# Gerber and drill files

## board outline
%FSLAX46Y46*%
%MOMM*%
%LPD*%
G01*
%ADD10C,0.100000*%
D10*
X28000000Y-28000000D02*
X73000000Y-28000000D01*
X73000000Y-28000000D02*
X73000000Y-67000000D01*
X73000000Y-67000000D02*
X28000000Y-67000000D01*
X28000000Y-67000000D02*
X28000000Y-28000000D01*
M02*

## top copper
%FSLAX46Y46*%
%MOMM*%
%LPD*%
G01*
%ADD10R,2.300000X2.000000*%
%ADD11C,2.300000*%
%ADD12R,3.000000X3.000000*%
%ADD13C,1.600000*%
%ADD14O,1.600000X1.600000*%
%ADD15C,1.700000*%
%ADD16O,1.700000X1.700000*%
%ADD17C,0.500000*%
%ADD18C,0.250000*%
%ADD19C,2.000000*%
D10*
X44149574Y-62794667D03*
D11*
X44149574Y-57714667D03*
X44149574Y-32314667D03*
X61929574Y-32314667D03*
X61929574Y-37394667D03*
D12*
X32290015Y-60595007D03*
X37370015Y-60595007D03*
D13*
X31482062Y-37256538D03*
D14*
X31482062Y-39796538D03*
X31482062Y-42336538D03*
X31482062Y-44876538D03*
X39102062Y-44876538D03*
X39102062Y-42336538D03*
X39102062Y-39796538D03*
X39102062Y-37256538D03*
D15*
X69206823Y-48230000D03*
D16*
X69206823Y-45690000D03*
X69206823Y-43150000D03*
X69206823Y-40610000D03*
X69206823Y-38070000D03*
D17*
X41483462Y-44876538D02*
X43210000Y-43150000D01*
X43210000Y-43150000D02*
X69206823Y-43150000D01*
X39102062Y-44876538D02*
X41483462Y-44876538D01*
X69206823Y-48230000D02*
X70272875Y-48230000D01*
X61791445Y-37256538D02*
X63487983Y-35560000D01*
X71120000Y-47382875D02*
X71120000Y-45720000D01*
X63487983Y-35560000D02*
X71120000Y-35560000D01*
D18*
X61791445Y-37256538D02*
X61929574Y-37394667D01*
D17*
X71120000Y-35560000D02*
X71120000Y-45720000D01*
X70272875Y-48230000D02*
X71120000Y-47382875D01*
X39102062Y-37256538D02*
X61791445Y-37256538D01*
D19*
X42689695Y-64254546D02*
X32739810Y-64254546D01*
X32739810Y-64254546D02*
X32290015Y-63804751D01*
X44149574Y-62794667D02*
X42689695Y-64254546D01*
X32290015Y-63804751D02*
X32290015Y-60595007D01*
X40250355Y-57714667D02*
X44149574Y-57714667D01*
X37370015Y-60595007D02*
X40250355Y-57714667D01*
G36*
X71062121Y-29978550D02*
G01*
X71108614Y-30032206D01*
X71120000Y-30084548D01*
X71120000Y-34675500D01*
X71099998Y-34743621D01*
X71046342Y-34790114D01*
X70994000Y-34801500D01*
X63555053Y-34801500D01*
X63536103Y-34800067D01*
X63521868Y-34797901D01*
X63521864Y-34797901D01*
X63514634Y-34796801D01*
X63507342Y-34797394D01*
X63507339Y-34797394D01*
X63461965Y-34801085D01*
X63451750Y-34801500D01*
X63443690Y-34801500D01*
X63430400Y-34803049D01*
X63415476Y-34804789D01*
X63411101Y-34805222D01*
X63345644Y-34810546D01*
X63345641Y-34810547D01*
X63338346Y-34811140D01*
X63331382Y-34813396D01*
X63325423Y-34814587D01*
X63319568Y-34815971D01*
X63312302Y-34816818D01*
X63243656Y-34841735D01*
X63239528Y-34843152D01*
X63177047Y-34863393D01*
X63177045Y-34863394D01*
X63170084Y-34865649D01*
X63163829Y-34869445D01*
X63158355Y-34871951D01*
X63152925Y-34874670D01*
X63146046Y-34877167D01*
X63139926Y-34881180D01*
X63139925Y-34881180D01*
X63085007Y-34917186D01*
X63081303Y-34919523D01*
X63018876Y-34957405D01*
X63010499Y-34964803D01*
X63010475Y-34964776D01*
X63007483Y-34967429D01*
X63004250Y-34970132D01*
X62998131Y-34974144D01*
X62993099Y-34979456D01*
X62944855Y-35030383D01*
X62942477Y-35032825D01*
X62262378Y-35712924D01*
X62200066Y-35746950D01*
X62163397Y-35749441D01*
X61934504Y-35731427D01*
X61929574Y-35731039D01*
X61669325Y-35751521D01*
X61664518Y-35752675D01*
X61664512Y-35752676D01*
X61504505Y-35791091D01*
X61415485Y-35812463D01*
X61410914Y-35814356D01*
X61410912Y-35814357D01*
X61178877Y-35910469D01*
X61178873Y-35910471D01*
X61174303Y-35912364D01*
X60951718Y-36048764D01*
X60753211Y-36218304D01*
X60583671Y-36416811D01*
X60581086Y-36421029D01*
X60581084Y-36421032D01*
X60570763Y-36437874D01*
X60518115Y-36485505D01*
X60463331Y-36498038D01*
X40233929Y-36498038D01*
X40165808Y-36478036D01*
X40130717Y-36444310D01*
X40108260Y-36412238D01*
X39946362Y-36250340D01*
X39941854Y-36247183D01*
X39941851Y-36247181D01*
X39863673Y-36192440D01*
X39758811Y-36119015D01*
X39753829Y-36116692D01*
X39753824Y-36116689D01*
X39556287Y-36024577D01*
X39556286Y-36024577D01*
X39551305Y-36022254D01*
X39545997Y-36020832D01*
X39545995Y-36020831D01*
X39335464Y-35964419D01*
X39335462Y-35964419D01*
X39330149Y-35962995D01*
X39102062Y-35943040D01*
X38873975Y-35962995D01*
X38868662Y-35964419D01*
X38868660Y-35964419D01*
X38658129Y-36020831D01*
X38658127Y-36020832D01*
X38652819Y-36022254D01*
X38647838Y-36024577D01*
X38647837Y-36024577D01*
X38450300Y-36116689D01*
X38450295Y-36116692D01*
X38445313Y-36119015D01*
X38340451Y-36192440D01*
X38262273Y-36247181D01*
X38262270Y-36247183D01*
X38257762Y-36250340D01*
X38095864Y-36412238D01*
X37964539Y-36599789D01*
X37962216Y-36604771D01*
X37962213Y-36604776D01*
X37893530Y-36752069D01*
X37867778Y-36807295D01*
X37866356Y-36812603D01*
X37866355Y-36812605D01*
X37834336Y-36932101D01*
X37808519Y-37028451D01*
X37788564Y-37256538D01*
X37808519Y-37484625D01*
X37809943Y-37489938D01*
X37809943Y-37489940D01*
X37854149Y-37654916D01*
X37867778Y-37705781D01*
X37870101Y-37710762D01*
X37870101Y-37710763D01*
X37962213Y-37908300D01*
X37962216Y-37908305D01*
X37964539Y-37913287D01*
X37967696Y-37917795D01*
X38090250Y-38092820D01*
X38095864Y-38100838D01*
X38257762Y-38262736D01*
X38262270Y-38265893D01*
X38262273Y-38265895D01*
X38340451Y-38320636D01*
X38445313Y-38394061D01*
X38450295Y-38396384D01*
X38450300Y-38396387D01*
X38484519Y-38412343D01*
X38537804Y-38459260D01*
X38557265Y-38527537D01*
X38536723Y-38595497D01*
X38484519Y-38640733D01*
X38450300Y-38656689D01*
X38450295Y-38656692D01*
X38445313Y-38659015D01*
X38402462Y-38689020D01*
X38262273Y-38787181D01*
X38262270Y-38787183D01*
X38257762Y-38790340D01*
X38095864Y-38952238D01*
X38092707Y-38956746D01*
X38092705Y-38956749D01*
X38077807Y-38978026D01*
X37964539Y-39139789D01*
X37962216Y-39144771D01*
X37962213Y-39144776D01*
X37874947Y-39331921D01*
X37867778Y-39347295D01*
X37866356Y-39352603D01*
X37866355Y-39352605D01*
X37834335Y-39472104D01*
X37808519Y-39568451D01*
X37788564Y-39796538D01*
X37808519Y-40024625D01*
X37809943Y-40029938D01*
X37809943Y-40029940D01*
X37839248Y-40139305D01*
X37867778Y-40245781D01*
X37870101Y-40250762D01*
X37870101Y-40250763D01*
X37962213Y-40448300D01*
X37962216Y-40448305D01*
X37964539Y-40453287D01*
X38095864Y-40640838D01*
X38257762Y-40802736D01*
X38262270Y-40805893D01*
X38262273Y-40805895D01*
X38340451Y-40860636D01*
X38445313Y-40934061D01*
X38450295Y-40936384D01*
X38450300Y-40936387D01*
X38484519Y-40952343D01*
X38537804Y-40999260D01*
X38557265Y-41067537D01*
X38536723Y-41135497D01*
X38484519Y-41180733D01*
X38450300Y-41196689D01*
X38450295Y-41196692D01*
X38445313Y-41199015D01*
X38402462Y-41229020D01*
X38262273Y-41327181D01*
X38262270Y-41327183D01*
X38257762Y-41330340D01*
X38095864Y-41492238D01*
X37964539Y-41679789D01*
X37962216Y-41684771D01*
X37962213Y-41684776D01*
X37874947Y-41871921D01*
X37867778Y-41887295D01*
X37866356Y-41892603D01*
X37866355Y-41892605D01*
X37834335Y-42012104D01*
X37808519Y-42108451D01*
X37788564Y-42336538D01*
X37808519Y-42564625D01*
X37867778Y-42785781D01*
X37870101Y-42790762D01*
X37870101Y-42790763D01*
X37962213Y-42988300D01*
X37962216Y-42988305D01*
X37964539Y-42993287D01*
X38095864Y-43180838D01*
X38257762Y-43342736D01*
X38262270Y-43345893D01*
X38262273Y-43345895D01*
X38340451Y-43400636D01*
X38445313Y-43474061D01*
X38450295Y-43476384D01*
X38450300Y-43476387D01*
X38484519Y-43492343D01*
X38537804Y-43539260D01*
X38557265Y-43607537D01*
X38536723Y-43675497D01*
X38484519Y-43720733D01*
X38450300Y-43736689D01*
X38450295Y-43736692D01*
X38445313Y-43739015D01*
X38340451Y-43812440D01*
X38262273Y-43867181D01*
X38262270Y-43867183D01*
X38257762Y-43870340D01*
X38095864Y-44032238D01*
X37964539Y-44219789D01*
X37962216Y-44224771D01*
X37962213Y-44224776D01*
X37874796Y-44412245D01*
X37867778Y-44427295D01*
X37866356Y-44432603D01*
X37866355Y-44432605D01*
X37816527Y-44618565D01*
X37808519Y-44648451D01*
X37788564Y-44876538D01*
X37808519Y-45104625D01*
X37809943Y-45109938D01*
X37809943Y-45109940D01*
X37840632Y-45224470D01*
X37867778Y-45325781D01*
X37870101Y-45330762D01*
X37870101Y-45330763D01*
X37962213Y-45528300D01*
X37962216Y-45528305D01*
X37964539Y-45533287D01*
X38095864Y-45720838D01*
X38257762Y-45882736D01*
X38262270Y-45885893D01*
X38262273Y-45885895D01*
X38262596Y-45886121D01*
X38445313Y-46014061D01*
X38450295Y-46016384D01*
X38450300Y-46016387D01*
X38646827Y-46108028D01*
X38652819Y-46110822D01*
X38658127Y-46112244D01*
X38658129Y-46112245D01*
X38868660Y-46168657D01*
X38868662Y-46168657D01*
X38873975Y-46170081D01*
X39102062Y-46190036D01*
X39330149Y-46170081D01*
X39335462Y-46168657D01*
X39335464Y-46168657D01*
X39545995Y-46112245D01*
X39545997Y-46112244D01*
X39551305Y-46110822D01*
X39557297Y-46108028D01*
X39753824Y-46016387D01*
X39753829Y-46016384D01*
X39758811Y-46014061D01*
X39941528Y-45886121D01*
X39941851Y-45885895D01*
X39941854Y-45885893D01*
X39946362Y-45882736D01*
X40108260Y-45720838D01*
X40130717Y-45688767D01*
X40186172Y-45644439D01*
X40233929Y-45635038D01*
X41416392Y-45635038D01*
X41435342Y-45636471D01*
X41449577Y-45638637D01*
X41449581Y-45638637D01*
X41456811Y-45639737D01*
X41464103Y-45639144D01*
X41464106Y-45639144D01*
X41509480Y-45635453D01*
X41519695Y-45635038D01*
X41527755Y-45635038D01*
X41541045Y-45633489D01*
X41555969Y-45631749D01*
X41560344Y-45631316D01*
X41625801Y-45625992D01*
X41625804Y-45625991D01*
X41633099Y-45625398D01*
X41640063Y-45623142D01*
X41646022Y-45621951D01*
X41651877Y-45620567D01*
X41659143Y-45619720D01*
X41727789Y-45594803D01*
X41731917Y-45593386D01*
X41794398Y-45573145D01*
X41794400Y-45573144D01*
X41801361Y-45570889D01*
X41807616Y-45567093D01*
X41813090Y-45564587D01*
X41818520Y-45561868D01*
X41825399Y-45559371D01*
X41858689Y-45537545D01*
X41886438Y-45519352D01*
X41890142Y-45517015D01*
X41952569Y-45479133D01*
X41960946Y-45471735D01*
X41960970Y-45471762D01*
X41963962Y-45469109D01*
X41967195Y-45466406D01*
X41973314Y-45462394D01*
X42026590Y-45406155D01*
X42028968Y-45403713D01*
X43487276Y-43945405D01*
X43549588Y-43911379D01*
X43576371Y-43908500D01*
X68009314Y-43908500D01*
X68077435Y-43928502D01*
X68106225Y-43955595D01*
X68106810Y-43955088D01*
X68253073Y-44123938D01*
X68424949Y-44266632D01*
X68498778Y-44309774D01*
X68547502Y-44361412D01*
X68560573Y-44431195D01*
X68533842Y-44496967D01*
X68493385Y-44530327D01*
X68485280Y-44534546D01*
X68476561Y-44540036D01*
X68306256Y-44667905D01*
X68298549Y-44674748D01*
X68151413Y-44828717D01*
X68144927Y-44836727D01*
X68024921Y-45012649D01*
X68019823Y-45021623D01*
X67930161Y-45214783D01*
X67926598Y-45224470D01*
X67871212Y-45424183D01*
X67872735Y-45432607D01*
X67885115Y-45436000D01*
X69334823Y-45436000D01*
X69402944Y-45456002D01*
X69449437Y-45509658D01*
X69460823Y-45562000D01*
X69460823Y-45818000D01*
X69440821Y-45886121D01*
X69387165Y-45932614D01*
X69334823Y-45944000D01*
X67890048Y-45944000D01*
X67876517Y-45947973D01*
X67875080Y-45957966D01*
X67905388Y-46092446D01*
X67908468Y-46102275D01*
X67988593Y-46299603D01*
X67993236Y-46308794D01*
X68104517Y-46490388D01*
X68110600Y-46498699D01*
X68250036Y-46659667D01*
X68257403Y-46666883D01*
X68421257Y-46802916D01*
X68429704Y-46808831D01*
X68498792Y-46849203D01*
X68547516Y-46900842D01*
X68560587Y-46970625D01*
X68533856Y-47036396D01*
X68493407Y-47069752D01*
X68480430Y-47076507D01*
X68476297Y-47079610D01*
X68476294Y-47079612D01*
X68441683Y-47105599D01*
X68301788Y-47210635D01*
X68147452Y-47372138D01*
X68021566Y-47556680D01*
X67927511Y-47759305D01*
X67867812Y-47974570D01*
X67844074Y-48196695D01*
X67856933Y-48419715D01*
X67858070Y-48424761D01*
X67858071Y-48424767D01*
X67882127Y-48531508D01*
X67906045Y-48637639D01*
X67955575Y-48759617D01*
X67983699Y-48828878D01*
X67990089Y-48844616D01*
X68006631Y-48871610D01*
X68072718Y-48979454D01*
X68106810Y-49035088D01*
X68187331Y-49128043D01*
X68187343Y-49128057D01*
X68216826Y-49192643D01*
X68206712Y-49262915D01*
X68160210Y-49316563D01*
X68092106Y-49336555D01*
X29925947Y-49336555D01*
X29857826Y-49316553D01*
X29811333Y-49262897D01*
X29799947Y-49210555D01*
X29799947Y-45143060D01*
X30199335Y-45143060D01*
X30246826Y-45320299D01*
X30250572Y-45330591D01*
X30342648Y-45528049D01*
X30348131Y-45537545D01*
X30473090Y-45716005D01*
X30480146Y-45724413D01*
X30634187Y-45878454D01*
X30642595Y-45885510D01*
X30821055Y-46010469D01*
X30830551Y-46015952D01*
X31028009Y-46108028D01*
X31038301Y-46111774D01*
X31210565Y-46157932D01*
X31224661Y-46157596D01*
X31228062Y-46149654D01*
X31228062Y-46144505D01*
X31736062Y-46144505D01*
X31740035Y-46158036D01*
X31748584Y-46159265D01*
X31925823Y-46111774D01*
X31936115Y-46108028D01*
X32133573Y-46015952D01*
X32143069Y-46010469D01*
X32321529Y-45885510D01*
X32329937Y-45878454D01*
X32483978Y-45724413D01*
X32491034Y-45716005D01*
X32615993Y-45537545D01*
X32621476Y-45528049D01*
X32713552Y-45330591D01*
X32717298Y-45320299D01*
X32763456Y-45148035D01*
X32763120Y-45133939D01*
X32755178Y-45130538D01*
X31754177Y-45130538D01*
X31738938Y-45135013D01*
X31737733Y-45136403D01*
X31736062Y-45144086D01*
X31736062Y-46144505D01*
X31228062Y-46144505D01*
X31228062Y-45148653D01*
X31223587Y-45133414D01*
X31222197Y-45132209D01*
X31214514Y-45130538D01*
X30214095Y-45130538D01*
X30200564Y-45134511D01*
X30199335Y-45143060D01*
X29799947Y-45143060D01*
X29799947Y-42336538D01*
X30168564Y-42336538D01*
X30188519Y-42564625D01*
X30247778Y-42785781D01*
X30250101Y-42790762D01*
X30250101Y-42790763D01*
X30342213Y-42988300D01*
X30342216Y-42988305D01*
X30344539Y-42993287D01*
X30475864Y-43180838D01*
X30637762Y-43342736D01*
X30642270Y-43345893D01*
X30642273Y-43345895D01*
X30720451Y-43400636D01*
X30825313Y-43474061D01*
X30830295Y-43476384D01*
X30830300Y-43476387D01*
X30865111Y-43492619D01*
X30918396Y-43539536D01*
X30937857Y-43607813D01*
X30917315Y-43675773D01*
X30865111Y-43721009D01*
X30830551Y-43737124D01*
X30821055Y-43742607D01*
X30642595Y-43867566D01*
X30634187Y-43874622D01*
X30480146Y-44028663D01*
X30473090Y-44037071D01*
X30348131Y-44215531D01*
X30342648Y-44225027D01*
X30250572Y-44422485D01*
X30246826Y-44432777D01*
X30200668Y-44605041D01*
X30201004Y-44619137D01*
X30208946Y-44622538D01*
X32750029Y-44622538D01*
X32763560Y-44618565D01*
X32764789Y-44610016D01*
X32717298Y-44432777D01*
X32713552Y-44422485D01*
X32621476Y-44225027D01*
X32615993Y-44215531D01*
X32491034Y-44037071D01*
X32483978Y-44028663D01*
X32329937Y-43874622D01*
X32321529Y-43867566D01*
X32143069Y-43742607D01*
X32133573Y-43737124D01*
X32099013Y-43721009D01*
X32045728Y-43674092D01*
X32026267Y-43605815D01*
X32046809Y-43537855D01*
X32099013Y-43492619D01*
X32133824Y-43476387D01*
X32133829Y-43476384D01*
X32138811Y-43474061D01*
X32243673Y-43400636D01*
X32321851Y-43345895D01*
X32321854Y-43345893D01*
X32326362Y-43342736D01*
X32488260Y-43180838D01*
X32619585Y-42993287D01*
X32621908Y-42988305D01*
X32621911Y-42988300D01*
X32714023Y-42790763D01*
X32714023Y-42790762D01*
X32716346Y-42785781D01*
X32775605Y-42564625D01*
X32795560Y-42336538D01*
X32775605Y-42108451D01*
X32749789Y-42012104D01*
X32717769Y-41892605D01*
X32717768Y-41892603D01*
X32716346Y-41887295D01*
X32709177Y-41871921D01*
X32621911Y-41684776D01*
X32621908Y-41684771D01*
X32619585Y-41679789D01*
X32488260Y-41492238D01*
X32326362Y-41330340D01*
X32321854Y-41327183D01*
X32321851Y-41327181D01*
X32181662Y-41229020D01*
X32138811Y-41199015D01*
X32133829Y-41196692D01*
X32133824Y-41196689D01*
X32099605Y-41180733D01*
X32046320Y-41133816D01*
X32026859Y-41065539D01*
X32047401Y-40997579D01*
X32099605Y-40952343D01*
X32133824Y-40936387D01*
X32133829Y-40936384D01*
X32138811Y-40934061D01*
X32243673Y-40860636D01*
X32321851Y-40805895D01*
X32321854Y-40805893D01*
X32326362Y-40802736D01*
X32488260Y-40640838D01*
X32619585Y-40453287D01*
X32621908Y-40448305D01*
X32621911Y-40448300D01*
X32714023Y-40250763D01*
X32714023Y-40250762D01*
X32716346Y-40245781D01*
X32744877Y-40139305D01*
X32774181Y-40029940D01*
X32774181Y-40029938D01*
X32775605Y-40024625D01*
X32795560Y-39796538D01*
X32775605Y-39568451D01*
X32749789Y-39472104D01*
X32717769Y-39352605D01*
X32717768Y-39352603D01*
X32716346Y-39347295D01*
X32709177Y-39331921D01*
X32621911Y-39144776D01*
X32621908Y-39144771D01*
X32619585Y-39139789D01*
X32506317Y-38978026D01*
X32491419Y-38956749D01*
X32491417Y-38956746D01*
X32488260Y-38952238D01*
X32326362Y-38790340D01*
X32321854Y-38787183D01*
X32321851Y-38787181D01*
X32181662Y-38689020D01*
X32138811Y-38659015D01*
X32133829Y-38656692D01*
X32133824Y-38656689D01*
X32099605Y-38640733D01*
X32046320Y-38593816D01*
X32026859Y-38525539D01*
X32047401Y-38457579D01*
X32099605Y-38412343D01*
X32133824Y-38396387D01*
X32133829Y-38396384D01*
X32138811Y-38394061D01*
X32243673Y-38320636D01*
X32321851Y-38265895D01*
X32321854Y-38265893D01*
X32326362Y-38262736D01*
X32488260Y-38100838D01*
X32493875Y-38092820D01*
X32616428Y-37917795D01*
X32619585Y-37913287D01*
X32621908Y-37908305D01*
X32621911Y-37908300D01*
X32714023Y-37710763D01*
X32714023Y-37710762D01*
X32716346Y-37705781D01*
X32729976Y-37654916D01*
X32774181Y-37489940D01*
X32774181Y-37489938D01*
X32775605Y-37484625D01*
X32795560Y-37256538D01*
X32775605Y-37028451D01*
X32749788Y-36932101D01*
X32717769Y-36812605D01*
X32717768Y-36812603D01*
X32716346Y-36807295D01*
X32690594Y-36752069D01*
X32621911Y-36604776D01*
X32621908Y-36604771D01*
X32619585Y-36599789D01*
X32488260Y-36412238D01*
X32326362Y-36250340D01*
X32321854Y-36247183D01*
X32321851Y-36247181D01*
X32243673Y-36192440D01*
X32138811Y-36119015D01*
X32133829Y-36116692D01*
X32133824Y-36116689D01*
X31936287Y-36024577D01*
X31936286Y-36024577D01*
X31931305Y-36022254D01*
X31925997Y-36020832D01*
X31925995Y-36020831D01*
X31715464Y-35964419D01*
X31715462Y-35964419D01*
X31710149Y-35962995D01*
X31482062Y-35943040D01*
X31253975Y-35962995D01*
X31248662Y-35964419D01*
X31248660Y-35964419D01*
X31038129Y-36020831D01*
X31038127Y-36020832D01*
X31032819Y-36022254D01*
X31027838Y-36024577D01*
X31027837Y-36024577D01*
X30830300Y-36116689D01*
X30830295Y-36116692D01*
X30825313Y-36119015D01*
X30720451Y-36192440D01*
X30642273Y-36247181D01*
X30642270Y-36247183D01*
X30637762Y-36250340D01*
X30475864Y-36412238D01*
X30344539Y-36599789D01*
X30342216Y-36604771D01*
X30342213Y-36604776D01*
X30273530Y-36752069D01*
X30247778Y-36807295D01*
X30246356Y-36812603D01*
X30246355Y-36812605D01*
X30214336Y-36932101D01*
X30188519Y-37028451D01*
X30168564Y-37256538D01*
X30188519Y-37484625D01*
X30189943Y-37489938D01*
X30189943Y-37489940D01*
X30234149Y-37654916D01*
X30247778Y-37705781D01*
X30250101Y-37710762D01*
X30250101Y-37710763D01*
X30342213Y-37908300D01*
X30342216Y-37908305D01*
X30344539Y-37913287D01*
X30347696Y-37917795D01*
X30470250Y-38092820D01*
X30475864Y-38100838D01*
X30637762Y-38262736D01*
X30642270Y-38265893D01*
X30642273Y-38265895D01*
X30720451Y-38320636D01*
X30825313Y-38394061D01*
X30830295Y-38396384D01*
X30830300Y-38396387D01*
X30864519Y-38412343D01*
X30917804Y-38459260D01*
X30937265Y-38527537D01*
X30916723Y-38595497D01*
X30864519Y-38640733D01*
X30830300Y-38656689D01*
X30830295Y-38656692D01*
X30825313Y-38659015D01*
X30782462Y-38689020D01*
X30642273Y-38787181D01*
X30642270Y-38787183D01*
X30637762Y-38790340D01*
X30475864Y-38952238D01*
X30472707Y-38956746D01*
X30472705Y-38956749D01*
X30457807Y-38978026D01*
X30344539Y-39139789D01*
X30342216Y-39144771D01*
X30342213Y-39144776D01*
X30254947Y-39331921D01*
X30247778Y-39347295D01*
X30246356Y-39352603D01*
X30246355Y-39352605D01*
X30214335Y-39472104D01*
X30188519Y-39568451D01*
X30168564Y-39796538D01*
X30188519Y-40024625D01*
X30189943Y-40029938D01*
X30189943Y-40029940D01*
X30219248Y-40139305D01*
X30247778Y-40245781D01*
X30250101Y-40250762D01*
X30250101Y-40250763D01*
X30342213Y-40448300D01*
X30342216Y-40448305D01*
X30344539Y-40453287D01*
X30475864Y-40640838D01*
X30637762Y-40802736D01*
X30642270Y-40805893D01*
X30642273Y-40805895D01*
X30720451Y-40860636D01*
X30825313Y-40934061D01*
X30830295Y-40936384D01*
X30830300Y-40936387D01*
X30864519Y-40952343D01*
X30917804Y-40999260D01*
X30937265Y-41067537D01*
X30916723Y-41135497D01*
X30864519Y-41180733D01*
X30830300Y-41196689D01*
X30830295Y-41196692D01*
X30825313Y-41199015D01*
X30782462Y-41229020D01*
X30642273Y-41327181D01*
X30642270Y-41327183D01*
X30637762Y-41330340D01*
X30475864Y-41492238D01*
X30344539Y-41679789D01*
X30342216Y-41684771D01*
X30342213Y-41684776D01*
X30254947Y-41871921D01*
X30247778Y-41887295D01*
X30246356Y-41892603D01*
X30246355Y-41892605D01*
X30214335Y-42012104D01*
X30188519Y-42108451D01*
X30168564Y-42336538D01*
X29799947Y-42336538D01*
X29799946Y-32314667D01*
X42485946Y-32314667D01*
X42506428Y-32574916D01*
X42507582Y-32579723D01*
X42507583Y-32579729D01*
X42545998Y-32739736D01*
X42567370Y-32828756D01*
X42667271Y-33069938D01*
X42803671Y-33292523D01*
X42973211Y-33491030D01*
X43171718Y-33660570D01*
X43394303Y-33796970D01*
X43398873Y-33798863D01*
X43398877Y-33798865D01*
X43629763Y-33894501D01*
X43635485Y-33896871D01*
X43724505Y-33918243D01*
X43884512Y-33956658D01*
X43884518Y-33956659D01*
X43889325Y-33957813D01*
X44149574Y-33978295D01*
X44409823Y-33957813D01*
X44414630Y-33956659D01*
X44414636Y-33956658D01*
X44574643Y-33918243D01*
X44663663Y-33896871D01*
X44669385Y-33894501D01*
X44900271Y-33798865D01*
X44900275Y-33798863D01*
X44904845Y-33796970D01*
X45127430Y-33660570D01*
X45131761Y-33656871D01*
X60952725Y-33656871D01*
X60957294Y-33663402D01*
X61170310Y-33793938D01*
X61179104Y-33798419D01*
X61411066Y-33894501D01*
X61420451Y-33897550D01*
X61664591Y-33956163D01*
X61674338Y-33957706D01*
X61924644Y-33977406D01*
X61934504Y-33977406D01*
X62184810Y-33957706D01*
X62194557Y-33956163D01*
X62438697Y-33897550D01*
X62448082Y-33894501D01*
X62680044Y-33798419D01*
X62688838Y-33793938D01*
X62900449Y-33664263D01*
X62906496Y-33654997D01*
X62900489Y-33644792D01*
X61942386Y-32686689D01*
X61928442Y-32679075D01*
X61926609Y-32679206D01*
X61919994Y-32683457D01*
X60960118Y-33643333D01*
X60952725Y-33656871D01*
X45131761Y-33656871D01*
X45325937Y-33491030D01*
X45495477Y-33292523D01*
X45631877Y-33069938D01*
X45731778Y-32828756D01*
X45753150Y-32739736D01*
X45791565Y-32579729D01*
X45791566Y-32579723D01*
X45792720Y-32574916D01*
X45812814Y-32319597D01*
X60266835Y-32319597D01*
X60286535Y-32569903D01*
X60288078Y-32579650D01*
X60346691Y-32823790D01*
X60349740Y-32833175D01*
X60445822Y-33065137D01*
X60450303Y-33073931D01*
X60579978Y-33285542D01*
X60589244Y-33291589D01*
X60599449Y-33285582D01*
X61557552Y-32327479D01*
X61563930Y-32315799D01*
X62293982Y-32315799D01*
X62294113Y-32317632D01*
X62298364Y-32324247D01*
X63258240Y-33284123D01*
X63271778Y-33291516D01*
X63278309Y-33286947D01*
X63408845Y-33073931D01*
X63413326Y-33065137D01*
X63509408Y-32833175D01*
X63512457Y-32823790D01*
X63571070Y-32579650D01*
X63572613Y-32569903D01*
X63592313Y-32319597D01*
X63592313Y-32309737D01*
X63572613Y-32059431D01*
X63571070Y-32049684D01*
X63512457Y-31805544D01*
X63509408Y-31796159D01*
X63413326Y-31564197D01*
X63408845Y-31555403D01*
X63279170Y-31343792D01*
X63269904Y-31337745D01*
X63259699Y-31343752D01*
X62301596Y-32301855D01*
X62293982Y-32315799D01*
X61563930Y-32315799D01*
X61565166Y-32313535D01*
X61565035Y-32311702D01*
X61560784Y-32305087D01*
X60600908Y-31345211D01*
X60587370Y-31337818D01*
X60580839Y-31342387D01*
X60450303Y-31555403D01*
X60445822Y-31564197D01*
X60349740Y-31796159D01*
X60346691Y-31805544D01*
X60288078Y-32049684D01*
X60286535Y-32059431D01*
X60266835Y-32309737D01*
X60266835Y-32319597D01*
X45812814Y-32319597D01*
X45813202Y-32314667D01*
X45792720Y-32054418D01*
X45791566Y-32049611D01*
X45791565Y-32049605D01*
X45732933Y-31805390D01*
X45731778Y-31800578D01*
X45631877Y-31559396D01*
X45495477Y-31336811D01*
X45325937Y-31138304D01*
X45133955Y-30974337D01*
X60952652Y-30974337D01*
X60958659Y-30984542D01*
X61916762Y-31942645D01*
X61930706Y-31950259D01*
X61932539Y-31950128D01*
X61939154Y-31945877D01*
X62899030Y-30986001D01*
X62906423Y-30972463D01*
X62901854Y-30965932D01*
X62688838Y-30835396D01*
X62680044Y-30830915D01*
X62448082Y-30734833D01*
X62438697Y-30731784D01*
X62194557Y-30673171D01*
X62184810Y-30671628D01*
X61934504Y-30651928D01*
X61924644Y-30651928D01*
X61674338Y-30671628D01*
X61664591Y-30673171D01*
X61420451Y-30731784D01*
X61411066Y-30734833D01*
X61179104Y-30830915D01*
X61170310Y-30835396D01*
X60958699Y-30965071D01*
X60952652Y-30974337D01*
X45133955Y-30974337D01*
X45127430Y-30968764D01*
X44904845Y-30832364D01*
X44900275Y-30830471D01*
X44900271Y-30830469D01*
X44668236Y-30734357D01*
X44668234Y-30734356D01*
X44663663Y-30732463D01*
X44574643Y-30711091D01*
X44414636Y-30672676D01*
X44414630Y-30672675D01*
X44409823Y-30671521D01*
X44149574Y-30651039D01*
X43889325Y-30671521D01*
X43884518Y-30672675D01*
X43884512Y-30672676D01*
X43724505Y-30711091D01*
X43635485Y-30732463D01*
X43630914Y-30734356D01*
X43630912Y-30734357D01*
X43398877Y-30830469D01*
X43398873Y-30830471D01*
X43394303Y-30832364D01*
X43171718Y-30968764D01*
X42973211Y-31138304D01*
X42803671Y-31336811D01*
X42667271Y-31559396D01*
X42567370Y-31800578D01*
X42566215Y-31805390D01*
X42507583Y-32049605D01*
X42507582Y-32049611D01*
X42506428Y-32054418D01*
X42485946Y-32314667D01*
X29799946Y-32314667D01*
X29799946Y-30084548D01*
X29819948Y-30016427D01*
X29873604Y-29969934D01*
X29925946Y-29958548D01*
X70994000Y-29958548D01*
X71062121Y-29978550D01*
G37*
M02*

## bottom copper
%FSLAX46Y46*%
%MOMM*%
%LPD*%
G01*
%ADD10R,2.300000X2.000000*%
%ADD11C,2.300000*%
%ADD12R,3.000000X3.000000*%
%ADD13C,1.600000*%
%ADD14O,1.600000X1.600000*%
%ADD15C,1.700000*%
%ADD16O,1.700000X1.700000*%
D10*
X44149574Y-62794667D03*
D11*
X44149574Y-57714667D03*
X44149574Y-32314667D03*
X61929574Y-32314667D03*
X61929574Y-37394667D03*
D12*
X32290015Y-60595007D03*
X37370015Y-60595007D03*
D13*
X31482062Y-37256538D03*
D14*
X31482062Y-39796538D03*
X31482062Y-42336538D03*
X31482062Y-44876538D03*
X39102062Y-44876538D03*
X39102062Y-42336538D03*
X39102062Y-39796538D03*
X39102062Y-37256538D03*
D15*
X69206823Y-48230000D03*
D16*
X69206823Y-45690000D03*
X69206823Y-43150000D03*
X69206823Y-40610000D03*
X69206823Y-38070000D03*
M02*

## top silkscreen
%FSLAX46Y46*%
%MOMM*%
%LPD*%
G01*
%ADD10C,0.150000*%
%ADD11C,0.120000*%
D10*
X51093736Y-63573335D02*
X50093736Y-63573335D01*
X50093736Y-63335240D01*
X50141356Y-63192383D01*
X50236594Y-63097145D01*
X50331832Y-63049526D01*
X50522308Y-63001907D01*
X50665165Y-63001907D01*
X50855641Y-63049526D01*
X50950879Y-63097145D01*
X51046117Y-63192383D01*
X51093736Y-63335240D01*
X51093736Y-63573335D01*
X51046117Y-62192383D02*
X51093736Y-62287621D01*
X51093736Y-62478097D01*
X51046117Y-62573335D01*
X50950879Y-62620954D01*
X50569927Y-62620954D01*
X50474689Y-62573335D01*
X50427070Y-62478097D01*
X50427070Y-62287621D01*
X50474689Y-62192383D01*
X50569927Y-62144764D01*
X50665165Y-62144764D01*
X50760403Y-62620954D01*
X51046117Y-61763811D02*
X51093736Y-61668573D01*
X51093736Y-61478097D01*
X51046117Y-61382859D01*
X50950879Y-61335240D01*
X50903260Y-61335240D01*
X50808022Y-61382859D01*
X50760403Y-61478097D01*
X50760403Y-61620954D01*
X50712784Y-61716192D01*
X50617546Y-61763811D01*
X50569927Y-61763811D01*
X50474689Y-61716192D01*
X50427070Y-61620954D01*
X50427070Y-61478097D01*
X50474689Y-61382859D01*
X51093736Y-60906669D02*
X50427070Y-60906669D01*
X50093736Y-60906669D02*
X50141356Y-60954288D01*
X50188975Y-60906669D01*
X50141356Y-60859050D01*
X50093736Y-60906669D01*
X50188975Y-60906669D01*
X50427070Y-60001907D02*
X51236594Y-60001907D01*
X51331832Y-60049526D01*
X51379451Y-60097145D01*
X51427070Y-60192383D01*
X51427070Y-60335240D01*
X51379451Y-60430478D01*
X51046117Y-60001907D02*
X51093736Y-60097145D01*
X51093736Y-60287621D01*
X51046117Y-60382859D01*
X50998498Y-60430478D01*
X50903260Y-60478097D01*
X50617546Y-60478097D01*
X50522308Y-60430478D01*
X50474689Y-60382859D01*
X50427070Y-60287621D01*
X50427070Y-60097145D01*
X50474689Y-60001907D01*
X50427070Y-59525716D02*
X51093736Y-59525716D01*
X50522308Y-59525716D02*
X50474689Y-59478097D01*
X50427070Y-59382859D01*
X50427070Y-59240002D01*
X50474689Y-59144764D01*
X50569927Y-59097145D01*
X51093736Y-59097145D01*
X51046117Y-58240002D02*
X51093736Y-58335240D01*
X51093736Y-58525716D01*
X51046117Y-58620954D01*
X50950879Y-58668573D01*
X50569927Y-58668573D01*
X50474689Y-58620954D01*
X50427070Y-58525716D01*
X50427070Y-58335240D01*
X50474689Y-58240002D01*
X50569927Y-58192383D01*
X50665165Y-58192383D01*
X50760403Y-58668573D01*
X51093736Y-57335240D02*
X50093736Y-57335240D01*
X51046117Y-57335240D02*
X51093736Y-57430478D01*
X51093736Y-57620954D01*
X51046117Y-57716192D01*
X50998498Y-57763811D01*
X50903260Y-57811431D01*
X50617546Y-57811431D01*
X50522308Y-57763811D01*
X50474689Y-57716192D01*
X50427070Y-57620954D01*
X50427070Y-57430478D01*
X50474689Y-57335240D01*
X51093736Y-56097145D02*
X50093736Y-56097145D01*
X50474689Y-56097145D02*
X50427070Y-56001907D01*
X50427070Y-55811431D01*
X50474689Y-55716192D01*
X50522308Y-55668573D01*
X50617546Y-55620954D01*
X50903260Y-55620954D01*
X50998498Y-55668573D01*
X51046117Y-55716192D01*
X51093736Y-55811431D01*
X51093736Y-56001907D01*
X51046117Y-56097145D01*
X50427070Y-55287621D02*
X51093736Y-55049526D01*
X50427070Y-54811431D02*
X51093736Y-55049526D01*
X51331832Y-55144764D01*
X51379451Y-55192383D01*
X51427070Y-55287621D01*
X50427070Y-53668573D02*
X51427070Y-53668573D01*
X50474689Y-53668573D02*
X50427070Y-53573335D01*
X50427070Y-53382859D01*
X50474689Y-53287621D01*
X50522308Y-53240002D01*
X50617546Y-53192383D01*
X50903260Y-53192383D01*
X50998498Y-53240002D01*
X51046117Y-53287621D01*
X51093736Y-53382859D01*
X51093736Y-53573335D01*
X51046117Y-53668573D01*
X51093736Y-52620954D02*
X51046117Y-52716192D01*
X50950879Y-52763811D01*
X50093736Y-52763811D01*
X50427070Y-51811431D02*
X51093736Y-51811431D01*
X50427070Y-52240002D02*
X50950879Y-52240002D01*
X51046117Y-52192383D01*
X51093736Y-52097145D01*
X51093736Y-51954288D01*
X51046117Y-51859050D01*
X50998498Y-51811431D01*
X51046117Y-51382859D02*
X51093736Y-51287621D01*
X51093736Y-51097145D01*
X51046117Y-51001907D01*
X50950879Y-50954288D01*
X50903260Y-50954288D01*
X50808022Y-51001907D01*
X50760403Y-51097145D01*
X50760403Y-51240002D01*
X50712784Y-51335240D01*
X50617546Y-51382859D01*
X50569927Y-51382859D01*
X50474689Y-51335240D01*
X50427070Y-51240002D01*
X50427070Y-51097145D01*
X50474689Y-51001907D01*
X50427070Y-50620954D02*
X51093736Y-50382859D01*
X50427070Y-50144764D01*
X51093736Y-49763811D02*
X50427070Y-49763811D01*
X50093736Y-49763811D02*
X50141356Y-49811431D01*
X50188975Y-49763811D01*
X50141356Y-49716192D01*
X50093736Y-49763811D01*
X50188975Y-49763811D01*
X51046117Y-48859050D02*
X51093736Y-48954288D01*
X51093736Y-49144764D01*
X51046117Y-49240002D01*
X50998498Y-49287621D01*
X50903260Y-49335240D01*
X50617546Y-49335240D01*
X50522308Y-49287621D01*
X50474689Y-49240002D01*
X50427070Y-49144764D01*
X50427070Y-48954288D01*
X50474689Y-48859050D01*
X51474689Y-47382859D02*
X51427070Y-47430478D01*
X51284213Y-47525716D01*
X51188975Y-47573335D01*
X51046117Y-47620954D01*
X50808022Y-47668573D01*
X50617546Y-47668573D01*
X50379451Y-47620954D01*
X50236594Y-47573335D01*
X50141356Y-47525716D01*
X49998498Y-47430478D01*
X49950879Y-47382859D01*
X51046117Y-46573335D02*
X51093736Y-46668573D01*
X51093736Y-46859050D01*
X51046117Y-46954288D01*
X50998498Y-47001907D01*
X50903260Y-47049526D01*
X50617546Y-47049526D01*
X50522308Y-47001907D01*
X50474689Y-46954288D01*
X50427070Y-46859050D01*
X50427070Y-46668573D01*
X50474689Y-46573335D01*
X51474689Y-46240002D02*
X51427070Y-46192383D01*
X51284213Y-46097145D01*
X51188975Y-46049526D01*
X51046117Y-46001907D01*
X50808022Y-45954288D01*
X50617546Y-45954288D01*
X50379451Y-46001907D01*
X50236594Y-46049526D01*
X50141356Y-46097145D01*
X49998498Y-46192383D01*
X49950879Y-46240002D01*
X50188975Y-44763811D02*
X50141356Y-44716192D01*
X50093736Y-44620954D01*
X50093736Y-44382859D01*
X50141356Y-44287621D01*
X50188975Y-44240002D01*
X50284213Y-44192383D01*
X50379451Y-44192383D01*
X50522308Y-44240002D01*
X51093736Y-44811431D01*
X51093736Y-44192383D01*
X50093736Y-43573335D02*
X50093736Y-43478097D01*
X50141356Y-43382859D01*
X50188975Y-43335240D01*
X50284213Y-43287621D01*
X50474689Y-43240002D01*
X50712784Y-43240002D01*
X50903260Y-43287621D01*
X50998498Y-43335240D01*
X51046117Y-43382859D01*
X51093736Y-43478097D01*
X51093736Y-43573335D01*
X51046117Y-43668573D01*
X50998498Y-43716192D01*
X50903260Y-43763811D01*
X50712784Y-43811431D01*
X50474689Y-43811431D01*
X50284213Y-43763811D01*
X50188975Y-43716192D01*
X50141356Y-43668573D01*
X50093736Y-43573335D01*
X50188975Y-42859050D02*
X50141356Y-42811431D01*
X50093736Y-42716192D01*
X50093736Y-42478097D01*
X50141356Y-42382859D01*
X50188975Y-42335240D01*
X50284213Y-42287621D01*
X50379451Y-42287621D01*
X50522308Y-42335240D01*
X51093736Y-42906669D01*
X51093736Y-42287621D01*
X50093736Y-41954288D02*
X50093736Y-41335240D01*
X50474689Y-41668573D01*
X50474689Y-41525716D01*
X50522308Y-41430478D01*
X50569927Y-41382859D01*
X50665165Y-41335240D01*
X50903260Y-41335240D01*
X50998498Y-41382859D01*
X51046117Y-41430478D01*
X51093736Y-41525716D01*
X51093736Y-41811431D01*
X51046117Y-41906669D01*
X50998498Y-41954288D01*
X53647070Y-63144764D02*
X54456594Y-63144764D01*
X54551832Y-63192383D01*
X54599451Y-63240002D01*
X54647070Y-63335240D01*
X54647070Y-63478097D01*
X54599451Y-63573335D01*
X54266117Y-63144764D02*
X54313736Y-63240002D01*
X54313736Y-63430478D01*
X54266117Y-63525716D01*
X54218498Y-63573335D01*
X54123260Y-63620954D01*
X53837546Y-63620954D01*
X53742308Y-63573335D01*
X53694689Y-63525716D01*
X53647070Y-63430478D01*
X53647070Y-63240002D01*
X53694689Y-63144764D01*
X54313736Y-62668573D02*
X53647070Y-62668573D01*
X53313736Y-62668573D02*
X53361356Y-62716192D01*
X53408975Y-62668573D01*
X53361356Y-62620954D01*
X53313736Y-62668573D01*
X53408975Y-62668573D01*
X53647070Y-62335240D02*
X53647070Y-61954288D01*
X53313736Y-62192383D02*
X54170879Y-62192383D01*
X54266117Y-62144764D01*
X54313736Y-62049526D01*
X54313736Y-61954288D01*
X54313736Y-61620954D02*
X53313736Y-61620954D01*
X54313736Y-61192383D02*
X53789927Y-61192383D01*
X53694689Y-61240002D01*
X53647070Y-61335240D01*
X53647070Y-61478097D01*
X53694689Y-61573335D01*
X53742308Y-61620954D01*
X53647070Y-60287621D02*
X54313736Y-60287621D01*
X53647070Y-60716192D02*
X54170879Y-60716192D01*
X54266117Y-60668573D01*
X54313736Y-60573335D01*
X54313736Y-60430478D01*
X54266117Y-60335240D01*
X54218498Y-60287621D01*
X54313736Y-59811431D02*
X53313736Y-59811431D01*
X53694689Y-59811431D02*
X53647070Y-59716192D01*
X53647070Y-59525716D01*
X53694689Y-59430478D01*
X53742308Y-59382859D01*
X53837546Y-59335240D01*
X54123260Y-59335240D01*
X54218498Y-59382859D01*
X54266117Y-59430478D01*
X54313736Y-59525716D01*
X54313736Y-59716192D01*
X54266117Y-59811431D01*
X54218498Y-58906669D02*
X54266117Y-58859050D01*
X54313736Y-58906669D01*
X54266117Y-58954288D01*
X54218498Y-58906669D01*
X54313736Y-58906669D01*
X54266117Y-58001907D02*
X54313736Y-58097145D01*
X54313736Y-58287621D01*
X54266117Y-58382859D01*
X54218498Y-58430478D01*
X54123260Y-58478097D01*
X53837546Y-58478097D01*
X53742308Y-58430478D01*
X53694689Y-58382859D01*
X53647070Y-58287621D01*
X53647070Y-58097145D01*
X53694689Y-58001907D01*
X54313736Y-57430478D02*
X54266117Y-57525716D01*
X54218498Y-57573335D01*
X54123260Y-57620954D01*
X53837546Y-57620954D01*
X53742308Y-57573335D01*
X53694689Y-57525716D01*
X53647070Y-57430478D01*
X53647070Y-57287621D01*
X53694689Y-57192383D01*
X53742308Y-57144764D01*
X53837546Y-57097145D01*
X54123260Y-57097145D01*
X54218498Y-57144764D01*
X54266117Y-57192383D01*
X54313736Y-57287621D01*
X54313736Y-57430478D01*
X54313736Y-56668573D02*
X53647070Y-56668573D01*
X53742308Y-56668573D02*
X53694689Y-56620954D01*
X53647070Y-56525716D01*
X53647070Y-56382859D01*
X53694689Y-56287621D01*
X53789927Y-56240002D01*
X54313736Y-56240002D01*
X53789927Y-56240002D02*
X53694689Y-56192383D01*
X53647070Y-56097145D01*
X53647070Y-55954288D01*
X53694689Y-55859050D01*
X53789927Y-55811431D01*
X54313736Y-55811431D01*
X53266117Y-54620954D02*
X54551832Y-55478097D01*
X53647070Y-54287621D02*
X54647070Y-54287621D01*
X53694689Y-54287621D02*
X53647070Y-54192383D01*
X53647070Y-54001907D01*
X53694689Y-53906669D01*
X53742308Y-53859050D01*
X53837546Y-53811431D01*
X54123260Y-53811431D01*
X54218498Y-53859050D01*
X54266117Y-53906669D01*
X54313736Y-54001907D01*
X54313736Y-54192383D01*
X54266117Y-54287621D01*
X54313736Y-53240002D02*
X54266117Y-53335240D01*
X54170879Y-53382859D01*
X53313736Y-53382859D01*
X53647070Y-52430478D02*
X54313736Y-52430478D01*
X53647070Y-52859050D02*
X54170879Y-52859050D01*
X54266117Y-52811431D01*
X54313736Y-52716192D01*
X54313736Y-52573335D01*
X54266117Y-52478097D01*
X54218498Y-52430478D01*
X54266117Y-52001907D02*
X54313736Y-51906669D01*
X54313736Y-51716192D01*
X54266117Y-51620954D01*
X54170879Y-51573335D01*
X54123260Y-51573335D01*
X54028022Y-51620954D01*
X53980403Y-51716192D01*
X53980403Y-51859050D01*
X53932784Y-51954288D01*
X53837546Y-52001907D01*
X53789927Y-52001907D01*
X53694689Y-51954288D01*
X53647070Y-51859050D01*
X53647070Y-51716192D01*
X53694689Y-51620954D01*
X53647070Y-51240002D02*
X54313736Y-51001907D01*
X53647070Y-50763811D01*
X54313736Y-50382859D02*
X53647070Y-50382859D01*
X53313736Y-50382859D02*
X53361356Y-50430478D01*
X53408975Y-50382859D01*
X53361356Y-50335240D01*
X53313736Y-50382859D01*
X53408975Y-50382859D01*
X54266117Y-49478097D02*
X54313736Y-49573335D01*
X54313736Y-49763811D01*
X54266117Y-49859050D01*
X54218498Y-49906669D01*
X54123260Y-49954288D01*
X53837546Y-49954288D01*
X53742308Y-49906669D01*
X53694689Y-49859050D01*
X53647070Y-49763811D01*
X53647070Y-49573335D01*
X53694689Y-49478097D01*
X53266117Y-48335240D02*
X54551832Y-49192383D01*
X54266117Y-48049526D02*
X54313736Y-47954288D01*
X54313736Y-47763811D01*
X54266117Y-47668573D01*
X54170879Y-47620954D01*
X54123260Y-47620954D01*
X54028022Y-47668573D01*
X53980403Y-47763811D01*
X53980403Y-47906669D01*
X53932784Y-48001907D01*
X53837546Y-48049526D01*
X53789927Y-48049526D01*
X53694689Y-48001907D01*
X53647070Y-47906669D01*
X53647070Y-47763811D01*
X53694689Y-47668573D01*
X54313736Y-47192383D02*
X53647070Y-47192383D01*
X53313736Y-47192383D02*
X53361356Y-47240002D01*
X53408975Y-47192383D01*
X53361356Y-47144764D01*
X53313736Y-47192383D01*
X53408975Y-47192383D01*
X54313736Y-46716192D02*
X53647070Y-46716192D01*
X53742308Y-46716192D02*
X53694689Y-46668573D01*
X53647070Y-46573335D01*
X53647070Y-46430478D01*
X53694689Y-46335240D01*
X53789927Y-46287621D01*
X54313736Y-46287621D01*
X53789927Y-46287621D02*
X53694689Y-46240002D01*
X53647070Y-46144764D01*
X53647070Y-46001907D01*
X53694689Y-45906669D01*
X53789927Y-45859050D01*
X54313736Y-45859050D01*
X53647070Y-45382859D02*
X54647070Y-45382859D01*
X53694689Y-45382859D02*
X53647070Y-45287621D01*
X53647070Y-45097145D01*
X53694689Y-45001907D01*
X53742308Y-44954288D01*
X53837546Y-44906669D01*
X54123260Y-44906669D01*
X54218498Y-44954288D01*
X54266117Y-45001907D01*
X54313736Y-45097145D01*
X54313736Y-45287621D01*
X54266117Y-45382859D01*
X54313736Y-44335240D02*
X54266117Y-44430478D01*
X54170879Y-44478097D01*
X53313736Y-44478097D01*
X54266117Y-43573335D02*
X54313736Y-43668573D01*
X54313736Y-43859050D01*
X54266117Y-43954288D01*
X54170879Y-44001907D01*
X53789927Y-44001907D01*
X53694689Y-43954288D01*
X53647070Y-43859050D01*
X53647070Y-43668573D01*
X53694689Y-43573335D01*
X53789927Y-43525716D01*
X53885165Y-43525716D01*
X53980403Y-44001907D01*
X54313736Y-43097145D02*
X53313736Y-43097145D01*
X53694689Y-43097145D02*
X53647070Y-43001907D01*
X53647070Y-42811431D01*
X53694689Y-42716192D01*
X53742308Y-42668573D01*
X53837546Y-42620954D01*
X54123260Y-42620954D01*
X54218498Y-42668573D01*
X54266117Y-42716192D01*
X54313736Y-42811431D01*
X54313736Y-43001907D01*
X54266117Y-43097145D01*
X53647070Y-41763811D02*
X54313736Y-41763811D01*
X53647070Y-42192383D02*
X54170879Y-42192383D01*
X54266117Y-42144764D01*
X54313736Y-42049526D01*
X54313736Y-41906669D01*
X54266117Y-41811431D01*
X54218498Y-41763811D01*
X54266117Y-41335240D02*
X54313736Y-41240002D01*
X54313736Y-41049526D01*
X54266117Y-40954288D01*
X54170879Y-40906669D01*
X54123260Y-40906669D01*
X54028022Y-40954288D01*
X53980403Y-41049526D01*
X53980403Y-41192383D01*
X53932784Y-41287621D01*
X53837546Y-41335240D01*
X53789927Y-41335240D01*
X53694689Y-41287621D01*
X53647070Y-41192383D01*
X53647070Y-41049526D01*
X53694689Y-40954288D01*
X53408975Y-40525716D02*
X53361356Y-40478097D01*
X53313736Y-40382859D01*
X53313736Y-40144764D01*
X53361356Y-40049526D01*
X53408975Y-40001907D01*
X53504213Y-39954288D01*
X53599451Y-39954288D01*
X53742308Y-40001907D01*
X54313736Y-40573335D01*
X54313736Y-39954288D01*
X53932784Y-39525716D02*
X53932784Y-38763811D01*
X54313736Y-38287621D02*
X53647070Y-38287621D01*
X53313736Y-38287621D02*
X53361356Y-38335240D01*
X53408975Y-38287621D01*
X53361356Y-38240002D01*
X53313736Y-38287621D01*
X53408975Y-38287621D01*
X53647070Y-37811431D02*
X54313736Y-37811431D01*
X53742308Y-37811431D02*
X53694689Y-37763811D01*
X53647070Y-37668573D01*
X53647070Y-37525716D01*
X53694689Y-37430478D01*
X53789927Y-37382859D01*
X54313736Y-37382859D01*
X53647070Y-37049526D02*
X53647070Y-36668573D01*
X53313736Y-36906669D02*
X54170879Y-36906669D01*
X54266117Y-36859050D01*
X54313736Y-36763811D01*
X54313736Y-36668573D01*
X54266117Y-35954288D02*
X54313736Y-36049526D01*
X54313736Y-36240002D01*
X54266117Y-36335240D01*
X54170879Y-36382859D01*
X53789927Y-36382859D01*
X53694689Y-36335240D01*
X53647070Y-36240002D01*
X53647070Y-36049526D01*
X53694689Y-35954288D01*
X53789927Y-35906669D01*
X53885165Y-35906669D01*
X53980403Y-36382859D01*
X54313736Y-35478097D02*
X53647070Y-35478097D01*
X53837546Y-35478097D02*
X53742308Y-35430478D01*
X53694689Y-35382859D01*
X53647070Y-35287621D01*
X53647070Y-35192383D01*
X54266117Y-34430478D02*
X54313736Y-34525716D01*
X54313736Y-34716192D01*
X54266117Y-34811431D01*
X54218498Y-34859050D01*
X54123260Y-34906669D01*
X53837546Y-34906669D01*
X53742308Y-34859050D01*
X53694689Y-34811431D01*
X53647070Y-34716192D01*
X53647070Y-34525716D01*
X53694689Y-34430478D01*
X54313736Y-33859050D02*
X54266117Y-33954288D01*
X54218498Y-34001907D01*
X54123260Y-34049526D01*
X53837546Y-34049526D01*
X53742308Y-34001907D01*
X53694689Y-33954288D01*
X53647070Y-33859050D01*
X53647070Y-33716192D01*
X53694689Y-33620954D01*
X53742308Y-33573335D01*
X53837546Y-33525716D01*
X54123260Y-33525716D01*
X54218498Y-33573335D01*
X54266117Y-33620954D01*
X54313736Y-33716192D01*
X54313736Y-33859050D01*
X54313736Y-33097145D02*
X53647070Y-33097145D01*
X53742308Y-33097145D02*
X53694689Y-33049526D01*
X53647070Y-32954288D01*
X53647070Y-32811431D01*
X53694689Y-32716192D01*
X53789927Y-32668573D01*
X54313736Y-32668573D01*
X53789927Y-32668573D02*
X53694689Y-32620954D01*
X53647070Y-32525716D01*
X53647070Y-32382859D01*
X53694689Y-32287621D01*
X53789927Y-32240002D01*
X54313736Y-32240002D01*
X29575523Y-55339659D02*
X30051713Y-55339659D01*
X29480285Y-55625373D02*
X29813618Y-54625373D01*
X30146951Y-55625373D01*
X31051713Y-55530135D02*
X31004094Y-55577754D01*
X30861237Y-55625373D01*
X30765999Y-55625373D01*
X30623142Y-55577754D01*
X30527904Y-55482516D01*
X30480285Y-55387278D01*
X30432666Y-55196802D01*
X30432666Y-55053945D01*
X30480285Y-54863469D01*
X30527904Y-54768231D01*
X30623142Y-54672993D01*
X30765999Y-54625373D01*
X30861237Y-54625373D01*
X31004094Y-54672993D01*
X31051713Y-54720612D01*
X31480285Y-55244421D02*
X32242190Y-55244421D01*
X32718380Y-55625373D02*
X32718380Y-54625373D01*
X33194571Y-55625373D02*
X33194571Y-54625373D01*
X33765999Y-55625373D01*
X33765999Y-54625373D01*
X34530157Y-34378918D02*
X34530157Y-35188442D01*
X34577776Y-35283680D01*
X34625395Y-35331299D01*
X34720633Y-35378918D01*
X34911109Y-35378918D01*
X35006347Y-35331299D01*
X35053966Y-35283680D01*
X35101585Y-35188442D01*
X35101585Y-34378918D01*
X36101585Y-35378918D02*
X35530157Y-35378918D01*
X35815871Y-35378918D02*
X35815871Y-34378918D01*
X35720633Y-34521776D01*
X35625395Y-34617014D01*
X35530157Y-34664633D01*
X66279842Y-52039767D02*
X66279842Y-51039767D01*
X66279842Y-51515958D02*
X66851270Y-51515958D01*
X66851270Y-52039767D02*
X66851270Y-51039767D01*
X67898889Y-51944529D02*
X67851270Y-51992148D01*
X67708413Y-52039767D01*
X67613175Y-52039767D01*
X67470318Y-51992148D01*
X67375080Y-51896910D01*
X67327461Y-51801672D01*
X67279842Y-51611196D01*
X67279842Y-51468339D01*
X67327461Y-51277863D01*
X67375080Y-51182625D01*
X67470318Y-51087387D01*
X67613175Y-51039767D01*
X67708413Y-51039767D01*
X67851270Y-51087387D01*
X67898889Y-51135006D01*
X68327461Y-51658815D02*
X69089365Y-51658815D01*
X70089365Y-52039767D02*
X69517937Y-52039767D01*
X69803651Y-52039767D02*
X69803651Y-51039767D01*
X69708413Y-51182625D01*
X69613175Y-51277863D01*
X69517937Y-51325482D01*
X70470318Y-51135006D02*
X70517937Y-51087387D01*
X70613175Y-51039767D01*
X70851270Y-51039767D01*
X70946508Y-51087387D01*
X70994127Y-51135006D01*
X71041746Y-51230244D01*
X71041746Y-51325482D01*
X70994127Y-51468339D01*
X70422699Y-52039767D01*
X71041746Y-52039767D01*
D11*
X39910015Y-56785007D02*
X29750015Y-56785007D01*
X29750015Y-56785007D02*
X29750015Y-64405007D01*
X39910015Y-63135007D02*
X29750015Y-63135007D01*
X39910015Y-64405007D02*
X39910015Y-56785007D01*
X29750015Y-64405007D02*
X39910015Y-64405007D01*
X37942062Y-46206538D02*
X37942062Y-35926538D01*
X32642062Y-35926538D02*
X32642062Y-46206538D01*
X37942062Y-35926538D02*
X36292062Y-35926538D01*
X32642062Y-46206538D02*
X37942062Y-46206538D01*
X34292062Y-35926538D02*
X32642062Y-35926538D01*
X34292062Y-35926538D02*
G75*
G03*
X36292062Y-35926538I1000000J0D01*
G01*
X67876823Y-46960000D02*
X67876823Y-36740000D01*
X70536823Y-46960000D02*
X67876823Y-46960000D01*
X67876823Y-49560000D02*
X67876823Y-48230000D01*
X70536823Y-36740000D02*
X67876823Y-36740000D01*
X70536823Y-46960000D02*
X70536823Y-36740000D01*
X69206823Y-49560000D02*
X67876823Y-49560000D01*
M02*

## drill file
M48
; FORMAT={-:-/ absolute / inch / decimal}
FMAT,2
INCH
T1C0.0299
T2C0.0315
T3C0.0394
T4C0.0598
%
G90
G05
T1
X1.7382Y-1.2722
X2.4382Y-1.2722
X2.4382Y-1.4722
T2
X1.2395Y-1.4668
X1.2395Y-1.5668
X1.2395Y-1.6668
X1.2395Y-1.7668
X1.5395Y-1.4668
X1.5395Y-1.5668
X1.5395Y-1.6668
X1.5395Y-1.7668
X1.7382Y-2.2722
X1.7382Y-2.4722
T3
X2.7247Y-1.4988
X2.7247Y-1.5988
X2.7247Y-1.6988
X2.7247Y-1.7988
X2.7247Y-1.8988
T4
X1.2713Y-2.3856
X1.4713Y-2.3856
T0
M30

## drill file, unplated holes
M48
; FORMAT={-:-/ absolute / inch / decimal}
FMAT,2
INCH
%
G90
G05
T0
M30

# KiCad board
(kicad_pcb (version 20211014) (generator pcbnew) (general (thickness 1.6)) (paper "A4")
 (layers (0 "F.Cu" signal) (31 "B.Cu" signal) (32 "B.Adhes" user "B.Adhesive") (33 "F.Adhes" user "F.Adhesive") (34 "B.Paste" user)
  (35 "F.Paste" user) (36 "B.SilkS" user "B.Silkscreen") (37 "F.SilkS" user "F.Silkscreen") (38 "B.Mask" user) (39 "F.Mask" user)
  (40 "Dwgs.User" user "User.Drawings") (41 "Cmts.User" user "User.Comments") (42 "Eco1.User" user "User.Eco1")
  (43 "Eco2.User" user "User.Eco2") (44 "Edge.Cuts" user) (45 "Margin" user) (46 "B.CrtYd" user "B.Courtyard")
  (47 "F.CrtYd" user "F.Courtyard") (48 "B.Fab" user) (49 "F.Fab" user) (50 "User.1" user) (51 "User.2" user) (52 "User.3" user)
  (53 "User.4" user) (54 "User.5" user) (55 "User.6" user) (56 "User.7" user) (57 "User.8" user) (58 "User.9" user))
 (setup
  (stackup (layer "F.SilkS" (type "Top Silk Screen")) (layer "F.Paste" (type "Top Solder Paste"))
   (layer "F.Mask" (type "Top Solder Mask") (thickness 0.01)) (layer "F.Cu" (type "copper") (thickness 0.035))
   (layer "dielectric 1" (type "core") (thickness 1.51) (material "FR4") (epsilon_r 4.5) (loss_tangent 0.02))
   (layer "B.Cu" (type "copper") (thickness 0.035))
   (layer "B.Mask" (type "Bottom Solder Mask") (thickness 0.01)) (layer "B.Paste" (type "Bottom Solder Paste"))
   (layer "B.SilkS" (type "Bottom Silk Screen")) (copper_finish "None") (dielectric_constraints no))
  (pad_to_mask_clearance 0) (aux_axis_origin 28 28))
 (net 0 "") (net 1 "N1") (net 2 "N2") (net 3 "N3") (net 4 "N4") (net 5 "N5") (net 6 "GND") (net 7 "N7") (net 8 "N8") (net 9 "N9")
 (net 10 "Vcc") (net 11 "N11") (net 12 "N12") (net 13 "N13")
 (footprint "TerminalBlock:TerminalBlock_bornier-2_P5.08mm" (layer "F.Cu") (at 32.290015 60.595007)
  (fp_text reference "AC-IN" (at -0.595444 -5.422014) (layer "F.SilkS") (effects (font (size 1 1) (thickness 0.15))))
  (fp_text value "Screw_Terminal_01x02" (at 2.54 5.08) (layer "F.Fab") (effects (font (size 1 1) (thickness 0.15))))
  (fp_line (start 7.62 -3.81) (end -2.54 -3.81) (layer "F.SilkS") (width 0.12))
  (fp_line (start -2.54 -3.81) (end -2.54 3.81) (layer "F.SilkS") (width 0.12))
  (fp_line (start 7.62 2.54) (end -2.54 2.54) (layer "F.SilkS") (width 0.12))
  (fp_line (start 7.62 3.81) (end 7.62 -3.81) (layer "F.SilkS") (width 0.12))
  (fp_line (start -2.54 3.81) (end 7.62 3.81) (layer "F.SilkS") (width 0.12))
  (pad "1" thru_hole rect (at 0 0) (size 3 3) (drill 1.52) (layers *.Cu *.Mask) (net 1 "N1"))
  (pad "2" thru_hole rect (at 5.08 0) (size 3 3) (drill 1.52) (layers *.Cu *.Mask) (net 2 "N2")))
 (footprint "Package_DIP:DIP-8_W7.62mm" (layer "F.Cu") (at 31.482062 37.256538)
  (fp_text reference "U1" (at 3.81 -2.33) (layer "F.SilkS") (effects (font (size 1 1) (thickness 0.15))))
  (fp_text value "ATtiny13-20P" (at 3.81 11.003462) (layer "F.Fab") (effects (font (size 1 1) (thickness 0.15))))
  (fp_line (start 6.46 8.95) (end 6.46 -1.33) (layer "F.SilkS") (width 0.12))
  (fp_line (start 1.16 -1.33) (end 1.16 8.95) (layer "F.SilkS") (width 0.12))
  (fp_line (start 6.46 -1.33) (end 4.81 -1.33) (layer "F.SilkS") (width 0.12))
  (fp_line (start 1.16 8.95) (end 6.46 8.95) (layer "F.SilkS") (width 0.12))
  (fp_line (start 2.81 -1.33) (end 1.16 -1.33) (layer "F.SilkS") (width 0.12))
  (fp_arc (start 4.81 -1.33) (mid 3.81 -0.33) (end 2.81 -1.33) (layer "F.SilkS") (width 0.12))
  (pad "1" thru_hole circle (at 0 0) (size 1.6 1.6) (drill 0.8) (layers *.Cu *.Mask) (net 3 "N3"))
  (pad "2" thru_hole oval (at 0 2.54) (size 1.6 1.6) (drill 0.8) (layers *.Cu *.Mask) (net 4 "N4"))
  (pad "3" thru_hole oval (at 0 5.08) (size 1.6 1.6) (drill 0.8) (layers *.Cu *.Mask) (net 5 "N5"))
  (pad "4" thru_hole oval (at 0 7.62) (size 1.6 1.6) (drill 0.8) (layers *.Cu *.Mask) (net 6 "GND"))
  (pad "5" thru_hole oval (at 7.62 7.62) (size 1.6 1.6) (drill 0.8) (layers *.Cu *.Mask) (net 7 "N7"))
  (pad "6" thru_hole oval (at 7.62 5.08) (size 1.6 1.6) (drill 0.8) (layers *.Cu *.Mask) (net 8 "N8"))
  (pad "7" thru_hole oval (at 7.62 2.54) (size 1.6 1.6) (drill 0.8) (layers *.Cu *.Mask) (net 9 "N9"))
  (pad "8" thru_hole oval (at 7.62 0) (size 1.6 1.6) (drill 0.8) (layers *.Cu *.Mask) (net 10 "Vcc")))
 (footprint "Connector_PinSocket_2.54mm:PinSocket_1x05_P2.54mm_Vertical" (layer "F.Cu") (at 69.206823 48.23 180)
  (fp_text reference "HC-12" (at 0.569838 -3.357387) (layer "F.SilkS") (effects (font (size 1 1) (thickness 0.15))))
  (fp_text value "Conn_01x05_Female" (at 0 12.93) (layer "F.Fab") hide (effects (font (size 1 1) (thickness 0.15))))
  (fp_line (start 1.33 1.27) (end 1.33 11.49) (layer "F.SilkS") (width 0.12))
  (fp_line (start -1.33 1.27) (end 1.33 1.27) (layer "F.SilkS") (width 0.12))
  (fp_line (start 1.33 -1.33) (end 1.33 0) (layer "F.SilkS") (width 0.12))
  (fp_line (start -1.33 11.49) (end 1.33 11.49) (layer "F.SilkS") (width 0.12))
  (fp_line (start -1.33 1.27) (end -1.33 11.49) (layer "F.SilkS") (width 0.12))
  (fp_line (start 0 -1.33) (end 1.33 -1.33) (layer "F.SilkS") (width 0.12))
  (pad "1" thru_hole circle (at 0 0 180) (size 1.7 1.7) (drill 1) (layers *.Cu *.Mask) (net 10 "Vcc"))
  (pad "2" thru_hole oval (at 0 2.54 180) (size 1.7 1.7) (drill 1) (layers *.Cu *.Mask) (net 6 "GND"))
  (pad "3" thru_hole oval (at 0 5.08 180) (size 1.7 1.7) (drill 1) (layers *.Cu *.Mask) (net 7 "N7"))
  (pad "4" thru_hole oval (at 0 7.62 180) (size 1.7 1.7) (drill 1) (layers *.Cu *.Mask) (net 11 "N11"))
  (pad "5" thru_hole oval (at 0 10.16 180) (size 1.7 1.7) (drill 1) (layers *.Cu *.Mask) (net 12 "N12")))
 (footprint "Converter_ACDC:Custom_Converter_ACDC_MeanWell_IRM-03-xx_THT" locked (layer "B.Cu") (at 44.149574 62.794667)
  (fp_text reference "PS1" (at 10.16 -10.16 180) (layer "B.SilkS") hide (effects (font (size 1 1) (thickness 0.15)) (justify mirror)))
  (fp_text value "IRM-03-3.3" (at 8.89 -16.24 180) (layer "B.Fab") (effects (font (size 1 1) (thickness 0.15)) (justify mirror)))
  (pad "1" thru_hole rect locked (at 0 0) (size 2.3 2) (drill 0.8) (layers *.Cu *.Mask) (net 1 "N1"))
  (pad "3" thru_hole circle locked (at 0 -5.08) (size 2.3 2.3) (drill 0.8) (layers *.Cu *.Mask) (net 2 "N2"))
  (pad "5" thru_hole circle locked (at 0 -30.48) (size 2.3 2.3) (drill 0.76) (layers *.Cu *.Mask) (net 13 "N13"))
  (pad "14" thru_hole circle locked (at 17.78 -30.48) (size 2.3 2.3) (drill 0.76) (layers *.Cu *.Mask) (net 6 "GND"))
  (pad "16" thru_hole circle locked (at 17.78 -25.4) (size 2.3 2.3) (drill 0.76) (layers *.Cu *.Mask) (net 10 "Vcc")))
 (gr_rect (start 28 28) (end 73 67) (layer "Edge.Cuts") (width 0.1) (fill none))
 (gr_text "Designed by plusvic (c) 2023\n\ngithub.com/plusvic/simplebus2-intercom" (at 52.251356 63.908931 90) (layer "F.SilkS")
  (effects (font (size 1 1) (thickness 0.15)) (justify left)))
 (segment (start 41.483462 44.876538) (end 43.21 43.15) (width 0.5) (layer "F.Cu") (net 7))
 (segment (start 43.21 43.15) (end 69.206823 43.15) (width 0.5) (layer "F.Cu") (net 7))
 (segment (start 39.102062 44.876538) (end 41.483462 44.876538) (width 0.5) (layer "F.Cu") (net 7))
 (segment (start 69.206823 48.23) (end 70.272875 48.23) (width 0.5) (layer "F.Cu") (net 10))
 (segment (start 61.791445 37.256538) (end 63.487983 35.56) (width 0.5) (layer "F.Cu") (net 10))
 (segment (start 71.12 47.382875) (end 71.12 45.72) (width 0.5) (layer "F.Cu") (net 10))
 (segment (start 63.487983 35.56) (end 71.12 35.56) (width 0.5) (layer "F.Cu") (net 10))
 (segment (start 61.791445 37.256538) (end 61.929574 37.394667) (width 0.25) (layer "F.Cu") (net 10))
 (segment (start 71.12 35.56) (end 71.12 45.72) (width 0.5) (layer "F.Cu") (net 10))
 (segment (start 70.272875 48.23) (end 71.12 47.382875) (width 0.5) (layer "F.Cu") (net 10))
 (segment (start 39.102062 37.256538) (end 61.791445 37.256538) (width 0.5) (layer "F.Cu") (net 10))
 (segment (start 42.689695 64.254546) (end 32.73981 64.254546) (width 2) (layer "F.Cu") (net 1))
 (segment (start 32.73981 64.254546) (end 32.290015 63.804751) (width 2) (layer "F.Cu") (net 1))
 (segment (start 44.149574 62.794667) (end 42.689695 64.254546) (width 2) (layer "F.Cu") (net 1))
 (segment (start 32.290015 63.804751) (end 32.290015 60.595007) (width 2) (layer "F.Cu") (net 1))
 (segment (start 40.250355 57.714667) (end 44.149574 57.714667) (width 2) (layer "F.Cu") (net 2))
 (segment (start 37.370015 60.595007) (end 40.250355 57.714667) (width 2) (layer "F.Cu") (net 2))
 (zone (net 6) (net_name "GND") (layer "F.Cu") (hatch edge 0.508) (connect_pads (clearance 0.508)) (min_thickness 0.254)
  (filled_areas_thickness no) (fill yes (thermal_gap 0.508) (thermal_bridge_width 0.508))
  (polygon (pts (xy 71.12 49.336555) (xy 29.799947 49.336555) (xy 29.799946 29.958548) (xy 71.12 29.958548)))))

